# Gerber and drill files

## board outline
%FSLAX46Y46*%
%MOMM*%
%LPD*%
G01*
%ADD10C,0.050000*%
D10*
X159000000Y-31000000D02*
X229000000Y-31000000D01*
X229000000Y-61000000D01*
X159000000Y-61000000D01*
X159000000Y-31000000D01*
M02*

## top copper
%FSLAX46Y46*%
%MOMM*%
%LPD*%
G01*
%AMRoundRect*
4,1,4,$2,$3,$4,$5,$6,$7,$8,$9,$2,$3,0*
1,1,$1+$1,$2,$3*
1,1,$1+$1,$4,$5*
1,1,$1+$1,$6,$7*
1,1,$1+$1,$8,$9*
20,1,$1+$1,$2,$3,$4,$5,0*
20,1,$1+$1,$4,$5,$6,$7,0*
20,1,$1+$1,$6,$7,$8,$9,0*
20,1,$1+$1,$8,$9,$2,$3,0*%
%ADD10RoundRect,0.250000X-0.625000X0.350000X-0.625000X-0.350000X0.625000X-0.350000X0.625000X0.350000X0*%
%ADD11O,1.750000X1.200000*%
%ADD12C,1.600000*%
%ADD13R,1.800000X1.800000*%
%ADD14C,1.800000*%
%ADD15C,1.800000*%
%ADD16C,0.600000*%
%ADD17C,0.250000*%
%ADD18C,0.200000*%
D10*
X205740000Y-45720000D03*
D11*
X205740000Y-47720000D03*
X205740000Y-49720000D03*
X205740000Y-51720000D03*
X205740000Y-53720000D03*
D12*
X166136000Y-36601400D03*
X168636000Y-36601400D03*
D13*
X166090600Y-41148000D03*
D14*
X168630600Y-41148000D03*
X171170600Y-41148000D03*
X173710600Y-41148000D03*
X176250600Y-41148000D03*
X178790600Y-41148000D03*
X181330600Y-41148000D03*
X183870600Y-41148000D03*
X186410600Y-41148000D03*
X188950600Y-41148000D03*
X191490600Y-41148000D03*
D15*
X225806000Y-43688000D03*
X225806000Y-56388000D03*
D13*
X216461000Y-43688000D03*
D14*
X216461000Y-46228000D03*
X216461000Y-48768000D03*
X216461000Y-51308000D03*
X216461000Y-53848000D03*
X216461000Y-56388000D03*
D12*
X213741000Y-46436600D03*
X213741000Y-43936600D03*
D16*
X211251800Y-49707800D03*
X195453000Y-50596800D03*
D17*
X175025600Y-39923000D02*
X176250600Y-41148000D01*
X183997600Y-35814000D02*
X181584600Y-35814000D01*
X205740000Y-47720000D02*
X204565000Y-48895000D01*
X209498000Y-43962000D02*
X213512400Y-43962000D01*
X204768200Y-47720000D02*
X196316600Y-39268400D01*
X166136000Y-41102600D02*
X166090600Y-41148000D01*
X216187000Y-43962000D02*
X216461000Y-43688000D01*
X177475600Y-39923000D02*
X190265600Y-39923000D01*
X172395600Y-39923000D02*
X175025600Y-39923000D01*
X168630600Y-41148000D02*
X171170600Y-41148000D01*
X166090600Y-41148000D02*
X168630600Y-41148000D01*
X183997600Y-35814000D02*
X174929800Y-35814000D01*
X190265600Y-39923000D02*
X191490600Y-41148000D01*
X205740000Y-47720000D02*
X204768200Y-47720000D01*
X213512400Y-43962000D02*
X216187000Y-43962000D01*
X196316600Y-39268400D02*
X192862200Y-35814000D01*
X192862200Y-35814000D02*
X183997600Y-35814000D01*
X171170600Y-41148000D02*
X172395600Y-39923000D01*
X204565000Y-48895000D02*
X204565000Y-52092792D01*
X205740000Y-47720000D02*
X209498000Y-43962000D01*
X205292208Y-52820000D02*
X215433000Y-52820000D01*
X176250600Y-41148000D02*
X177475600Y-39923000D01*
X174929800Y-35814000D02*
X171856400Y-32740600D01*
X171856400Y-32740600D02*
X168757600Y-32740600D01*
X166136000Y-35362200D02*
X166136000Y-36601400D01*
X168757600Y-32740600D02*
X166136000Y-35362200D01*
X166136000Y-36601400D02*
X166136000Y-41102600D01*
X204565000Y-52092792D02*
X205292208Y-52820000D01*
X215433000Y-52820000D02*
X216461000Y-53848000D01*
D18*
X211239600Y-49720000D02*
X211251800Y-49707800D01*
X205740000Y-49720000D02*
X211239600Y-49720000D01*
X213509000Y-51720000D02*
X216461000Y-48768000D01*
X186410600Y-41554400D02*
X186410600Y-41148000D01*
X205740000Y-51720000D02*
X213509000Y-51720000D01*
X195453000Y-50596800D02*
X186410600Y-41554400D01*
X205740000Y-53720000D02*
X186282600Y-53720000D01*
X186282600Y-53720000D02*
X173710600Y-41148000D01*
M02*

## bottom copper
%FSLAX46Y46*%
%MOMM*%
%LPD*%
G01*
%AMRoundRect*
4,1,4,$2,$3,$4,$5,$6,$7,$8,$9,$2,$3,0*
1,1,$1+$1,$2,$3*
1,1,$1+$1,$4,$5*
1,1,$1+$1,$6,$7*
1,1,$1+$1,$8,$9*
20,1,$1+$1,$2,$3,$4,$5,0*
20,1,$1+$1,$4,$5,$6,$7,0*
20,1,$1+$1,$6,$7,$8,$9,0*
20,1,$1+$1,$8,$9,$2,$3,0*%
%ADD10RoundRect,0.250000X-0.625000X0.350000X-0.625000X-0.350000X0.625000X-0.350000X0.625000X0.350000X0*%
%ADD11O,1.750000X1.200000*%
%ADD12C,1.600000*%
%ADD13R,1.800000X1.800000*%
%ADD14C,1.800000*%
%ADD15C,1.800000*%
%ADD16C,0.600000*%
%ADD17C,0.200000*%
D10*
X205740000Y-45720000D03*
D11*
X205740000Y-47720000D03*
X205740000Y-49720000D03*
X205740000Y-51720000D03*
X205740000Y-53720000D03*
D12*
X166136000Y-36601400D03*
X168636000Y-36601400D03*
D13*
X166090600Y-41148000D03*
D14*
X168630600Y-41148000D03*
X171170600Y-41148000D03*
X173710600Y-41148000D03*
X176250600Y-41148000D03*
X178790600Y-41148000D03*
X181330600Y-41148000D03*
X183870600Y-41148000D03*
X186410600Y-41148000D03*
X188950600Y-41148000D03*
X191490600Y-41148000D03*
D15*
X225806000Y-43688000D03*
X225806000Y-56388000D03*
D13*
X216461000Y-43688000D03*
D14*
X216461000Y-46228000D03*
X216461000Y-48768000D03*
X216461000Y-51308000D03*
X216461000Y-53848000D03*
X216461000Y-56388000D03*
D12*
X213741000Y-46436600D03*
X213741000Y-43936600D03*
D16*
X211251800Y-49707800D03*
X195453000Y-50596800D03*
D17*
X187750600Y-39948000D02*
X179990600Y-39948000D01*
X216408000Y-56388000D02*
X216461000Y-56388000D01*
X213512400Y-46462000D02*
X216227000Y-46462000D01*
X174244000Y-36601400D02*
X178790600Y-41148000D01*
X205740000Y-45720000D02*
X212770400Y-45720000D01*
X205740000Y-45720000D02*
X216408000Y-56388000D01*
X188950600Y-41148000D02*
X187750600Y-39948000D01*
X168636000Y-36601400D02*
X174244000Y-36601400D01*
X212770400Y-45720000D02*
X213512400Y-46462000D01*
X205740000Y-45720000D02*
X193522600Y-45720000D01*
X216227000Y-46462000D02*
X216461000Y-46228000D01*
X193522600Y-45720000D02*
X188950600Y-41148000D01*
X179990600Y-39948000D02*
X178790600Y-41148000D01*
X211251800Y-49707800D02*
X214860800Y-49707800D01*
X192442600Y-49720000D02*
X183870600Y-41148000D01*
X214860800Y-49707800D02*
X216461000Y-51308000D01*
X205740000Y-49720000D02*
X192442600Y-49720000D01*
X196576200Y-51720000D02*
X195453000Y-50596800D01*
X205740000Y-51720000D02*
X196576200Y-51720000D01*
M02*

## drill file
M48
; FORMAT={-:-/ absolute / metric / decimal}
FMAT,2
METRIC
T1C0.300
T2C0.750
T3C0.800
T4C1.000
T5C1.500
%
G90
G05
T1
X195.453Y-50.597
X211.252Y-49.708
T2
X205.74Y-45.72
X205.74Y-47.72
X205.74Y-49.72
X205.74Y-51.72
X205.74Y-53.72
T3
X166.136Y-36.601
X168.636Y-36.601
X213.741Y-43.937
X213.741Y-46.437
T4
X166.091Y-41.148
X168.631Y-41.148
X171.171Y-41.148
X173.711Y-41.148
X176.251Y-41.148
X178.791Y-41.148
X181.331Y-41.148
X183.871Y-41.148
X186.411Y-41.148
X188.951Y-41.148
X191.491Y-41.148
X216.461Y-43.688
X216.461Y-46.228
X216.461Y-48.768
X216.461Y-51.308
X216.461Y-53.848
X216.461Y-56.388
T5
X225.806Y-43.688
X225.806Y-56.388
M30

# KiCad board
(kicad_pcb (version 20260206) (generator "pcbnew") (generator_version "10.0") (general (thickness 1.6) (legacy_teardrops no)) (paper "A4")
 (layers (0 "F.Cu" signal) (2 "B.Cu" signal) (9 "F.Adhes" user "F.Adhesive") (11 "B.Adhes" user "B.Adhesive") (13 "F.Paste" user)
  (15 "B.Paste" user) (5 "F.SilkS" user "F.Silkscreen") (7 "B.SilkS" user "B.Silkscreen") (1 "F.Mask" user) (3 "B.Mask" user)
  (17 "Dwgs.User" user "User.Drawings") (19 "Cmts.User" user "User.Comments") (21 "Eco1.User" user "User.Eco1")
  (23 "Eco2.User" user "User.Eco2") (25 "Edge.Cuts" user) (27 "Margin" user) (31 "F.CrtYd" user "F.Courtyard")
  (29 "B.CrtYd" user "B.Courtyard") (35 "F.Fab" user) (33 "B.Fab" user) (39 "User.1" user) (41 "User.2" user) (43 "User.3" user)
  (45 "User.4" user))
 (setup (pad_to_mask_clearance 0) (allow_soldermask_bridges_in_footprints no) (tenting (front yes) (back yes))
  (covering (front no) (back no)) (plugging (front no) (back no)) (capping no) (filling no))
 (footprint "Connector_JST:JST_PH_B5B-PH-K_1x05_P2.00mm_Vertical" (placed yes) (layer "F.Cu") (at 205.74 45.72 -90)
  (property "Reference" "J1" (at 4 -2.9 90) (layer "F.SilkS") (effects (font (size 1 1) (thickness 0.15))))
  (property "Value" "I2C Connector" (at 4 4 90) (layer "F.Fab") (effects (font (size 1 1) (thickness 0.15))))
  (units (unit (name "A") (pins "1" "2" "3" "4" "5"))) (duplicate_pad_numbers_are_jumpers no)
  (pad "1" thru_hole roundrect (at 0 0 270) (size 1.2 1.75) (drill 0.75) (layers "*.Cu" "*.Mask") (remove_unused_layers no)
   (roundrect_rratio 0.208333) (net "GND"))
  (pad "2" thru_hole oval (at 2 0 270) (size 1.2 1.75) (drill 0.75) (layers "*.Cu" "*.Mask") (remove_unused_layers no) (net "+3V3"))
  (pad "3" thru_hole oval (at 4 0 270) (size 1.2 1.75) (drill 0.75) (layers "*.Cu" "*.Mask") (remove_unused_layers no) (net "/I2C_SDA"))
  (pad "4" thru_hole oval (at 6 0 270) (size 1.2 1.75) (drill 0.75) (layers "*.Cu" "*.Mask") (remove_unused_layers no) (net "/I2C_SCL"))
  (pad "5" thru_hole oval (at 8 0 270) (size 1.2 1.75) (drill 0.75) (layers "*.Cu" "*.Mask") (remove_unused_layers no) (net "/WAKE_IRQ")))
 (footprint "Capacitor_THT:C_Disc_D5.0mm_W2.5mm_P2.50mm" (layer "F.Cu") (at 166.136 36.6014)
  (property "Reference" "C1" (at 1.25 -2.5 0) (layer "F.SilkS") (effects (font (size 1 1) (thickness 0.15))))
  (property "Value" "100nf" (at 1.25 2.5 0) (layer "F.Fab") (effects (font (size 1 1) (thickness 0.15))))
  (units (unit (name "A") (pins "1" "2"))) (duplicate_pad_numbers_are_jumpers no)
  (pad "1" thru_hole circle (at 0 0) (size 1.6 1.6) (drill 0.8) (layers "*.Cu" "*.Mask") (remove_unused_layers no) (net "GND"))
  (pad "2" thru_hole circle (at 2.5 0) (size 1.6 1.6) (drill 0.8) (layers "*.Cu" "*.Mask") (remove_unused_layers no) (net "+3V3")))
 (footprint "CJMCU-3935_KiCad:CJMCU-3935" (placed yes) (layer "F.Cu") (at 178.7906 41.148)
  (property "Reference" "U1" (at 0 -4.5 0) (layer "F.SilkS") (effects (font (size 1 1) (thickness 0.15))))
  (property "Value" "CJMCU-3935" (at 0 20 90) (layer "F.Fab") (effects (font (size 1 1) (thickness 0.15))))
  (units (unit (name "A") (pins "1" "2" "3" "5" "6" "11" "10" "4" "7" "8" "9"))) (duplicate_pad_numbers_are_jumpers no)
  (pad "1" thru_hole rect (at -12.7 0) (size 1.8 1.8) (drill 1) (layers "*.Cu" "*.Mask") (remove_unused_layers no) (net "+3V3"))
  (pad "2" thru_hole circle (at -10.16 0) (size 1.8 1.8) (drill 1) (layers "*.Cu" "*.Mask") (remove_unused_layers no) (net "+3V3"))
  (pad "3" thru_hole circle (at -7.62 0) (size 1.8 1.8) (drill 1) (layers "*.Cu" "*.Mask") (remove_unused_layers no) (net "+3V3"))
  (pad "4" thru_hole circle (at -5.08 0) (size 1.8 1.8) (drill 1) (layers "*.Cu" "*.Mask") (remove_unused_layers no) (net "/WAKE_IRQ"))
  (pad "5" thru_hole circle (at -2.54 0) (size 1.8 1.8) (drill 1) (layers "*.Cu" "*.Mask") (remove_unused_layers no) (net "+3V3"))
  (pad "6" thru_hole circle (at 0 0) (size 1.8 1.8) (drill 1) (layers "*.Cu" "*.Mask") (remove_unused_layers no) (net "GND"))
  (pad "7" thru_hole circle (at 2.54 0) (size 1.8 1.8) (drill 1) (layers "*.Cu" "*.Mask") (remove_unused_layers no)
   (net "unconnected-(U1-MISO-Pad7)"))
  (pad "8" thru_hole circle (at 5.08 0) (size 1.8 1.8) (drill 1) (layers "*.Cu" "*.Mask") (remove_unused_layers no) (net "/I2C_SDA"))
  (pad "9" thru_hole circle (at 7.62 0) (size 1.8 1.8) (drill 1) (layers "*.Cu" "*.Mask") (remove_unused_layers no) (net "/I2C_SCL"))
  (pad "10" thru_hole circle (at 10.16 0) (size 1.8 1.8) (drill 1) (layers "*.Cu" "*.Mask") (remove_unused_layers no) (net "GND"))
  (pad "11" thru_hole circle (at 12.7 0) (size 1.8 1.8) (drill 1) (layers "*.Cu" "*.Mask") (remove_unused_layers no) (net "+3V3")))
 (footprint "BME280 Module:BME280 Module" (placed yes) (layer "F.Cu") (at 216.461 43.688 -90)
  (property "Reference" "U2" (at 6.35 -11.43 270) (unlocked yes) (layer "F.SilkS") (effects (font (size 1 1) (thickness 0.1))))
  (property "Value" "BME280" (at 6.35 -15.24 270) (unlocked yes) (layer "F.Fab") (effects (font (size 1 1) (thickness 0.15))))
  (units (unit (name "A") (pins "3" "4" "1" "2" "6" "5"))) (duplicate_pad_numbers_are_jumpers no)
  (pad "" np_thru_hole circle (at 0 -9.345 270) (size 1.8 1.8) (drill 1.5) (layers "*.Cu" "*.Mask"))
  (pad "" np_thru_hole circle (at 12.7 -9.345 270) (size 1.8 1.8) (drill 1.5) (layers "*.Cu" "*.Mask"))
  (pad "1" thru_hole rect (at 0 0 270) (size 1.8 1.8) (drill 1) (layers "*.Cu" "*.Mask") (remove_unused_layers no) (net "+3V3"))
  (pad "2" thru_hole circle (at 2.54 0 270) (size 1.8 1.8) (drill 1) (layers "*.Cu" "*.Mask") (remove_unused_layers no) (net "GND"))
  (pad "3" thru_hole circle (at 5.08 0 270) (size 1.8 1.8) (drill 1) (layers "*.Cu" "*.Mask") (remove_unused_layers no) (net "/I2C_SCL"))
  (pad "4" thru_hole circle (at 7.62 0 270) (size 1.8 1.8) (drill 1) (layers "*.Cu" "*.Mask") (remove_unused_layers no) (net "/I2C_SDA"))
  (pad "5" thru_hole circle (at 10.16 0 270) (size 1.8 1.8) (drill 1) (layers "*.Cu" "*.Mask") (remove_unused_layers no) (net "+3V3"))
  (pad "6" thru_hole circle (at 12.7 0 270) (size 1.8 1.8) (drill 1) (layers "*.Cu" "*.Mask") (remove_unused_layers no) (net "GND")))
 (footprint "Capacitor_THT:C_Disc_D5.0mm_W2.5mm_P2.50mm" (layer "F.Cu") (at 213.741 46.4366 90)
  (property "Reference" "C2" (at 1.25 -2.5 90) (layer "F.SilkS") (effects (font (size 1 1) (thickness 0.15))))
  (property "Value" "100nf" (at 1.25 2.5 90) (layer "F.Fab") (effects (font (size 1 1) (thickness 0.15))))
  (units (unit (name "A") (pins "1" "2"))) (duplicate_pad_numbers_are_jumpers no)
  (pad "1" thru_hole circle (at 0 0 90) (size 1.6 1.6) (drill 0.8) (layers "*.Cu" "*.Mask") (remove_unused_layers no) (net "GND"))
  (pad "2" thru_hole circle (at 2.5 0 90) (size 1.6 1.6) (drill 0.8) (layers "*.Cu" "*.Mask") (remove_unused_layers no) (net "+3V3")))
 (gr_rect (start 159 31) (end 229 61) (stroke (width 0.05) (type default)) (fill no) (layer "Edge.Cuts"))
 (segment (start 187.7506 39.948) (end 179.9906 39.948) (width 0.2) (layer "B.Cu") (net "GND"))
 (segment (start 216.408 56.388) (end 216.461 56.388) (width 0.2) (layer "B.Cu") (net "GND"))
 (segment (start 213.5124 46.462) (end 216.227 46.462) (width 0.2) (layer "B.Cu") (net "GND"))
 (segment (start 174.244 36.6014) (end 178.7906 41.148) (width 0.2) (layer "B.Cu") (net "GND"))
 (segment (start 205.74 45.72) (end 212.7704 45.72) (width 0.2) (layer "B.Cu") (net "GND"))
 (segment (start 205.74 45.72) (end 216.408 56.388) (width 0.2) (layer "B.Cu") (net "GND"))
 (segment (start 188.9506 41.148) (end 187.7506 39.948) (width 0.2) (layer "B.Cu") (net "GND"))
 (segment (start 168.636 36.6014) (end 174.244 36.6014) (width 0.2) (layer "B.Cu") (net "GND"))
 (segment (start 212.7704 45.72) (end 213.5124 46.462) (width 0.2) (layer "B.Cu") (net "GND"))
 (segment (start 205.74 45.72) (end 193.5226 45.72) (width 0.2) (layer "B.Cu") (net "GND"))
 (segment (start 216.227 46.462) (end 216.461 46.228) (width 0.2) (layer "B.Cu") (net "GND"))
 (segment (start 193.5226 45.72) (end 188.9506 41.148) (width 0.2) (layer "B.Cu") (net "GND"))
 (segment (start 179.9906 39.948) (end 178.7906 41.148) (width 0.2) (layer "B.Cu") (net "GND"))
 (segment (start 175.0256 39.923) (end 176.2506 41.148) (width 0.25) (layer "F.Cu") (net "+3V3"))
 (segment (start 183.9976 35.814) (end 181.5846 35.814) (width 0.25) (layer "F.Cu") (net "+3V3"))
 (segment (start 205.74 47.72) (end 204.565 48.895) (width 0.25) (layer "F.Cu") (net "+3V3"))
 (segment (start 209.498 43.962) (end 213.5124 43.962) (width 0.25) (layer "F.Cu") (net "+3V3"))
 (segment (start 204.7682 47.72) (end 196.3166 39.2684) (width 0.25) (layer "F.Cu") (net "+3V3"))
 (segment (start 166.136 41.1026) (end 166.0906 41.148) (width 0.25) (layer "F.Cu") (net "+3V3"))
 (segment (start 216.187 43.962) (end 216.461 43.688) (width 0.25) (layer "F.Cu") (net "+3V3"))
 (segment (start 177.4756 39.923) (end 190.2656 39.923) (width 0.25) (layer "F.Cu") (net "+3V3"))
 (segment (start 172.3956 39.923) (end 175.0256 39.923) (width 0.25) (layer "F.Cu") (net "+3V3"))
 (segment (start 168.6306 41.148) (end 171.1706 41.148) (width 0.25) (layer "F.Cu") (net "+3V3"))
 (segment (start 166.0906 41.148) (end 168.6306 41.148) (width 0.25) (layer "F.Cu") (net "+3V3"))
 (segment (start 183.9976 35.814) (end 174.9298 35.814) (width 0.25) (layer "F.Cu") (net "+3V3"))
 (segment (start 190.2656 39.923) (end 191.4906 41.148) (width 0.25) (layer "F.Cu") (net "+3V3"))
 (segment (start 205.74 47.72) (end 204.7682 47.72) (width 0.25) (layer "F.Cu") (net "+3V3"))
 (segment (start 213.5124 43.962) (end 216.187 43.962) (width 0.25) (layer "F.Cu") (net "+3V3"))
 (segment (start 196.3166 39.2684) (end 192.8622 35.814) (width 0.25) (layer "F.Cu") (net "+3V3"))
 (segment (start 192.8622 35.814) (end 183.9976 35.814) (width 0.25) (layer "F.Cu") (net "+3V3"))
 (segment (start 171.1706 41.148) (end 172.3956 39.923) (width 0.25) (layer "F.Cu") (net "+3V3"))
 (segment (start 204.565 48.895) (end 204.565 52.092792) (width 0.25) (layer "F.Cu") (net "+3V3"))
 (segment (start 205.74 47.72) (end 209.498 43.962) (width 0.25) (layer "F.Cu") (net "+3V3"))
 (segment (start 205.292208 52.82) (end 215.433 52.82) (width 0.25) (layer "F.Cu") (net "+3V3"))
 (segment (start 176.2506 41.148) (end 177.4756 39.923) (width 0.25) (layer "F.Cu") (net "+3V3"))
 (segment (start 174.9298 35.814) (end 171.8564 32.7406) (width 0.25) (layer "F.Cu") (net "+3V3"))
 (segment (start 171.8564 32.7406) (end 168.7576 32.7406) (width 0.25) (layer "F.Cu") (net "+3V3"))
 (segment (start 166.136 35.3622) (end 166.136 36.6014) (width 0.25) (layer "F.Cu") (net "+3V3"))
 (segment (start 168.7576 32.7406) (end 166.136 35.3622) (width 0.25) (layer "F.Cu") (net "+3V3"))
 (segment (start 166.136 36.6014) (end 166.136 41.1026) (width 0.25) (layer "F.Cu") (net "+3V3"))
 (segment (start 204.565 52.092792) (end 205.292208 52.82) (width 0.25) (layer "F.Cu") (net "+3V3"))
 (segment (start 215.433 52.82) (end 216.461 53.848) (width 0.25) (layer "F.Cu") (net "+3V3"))
 (segment (start 211.2396 49.72) (end 211.2518 49.7078) (width 0.2) (layer "F.Cu") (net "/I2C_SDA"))
 (segment (start 205.74 49.72) (end 211.2396 49.72) (width 0.2) (layer "F.Cu") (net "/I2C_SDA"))
 (via (at 211.2518 49.7078) (size 0.6) (drill 0.3) (layers "F.Cu" "B.Cu") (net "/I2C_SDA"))
 (segment (start 211.2518 49.7078) (end 214.8608 49.7078) (width 0.2) (layer "B.Cu") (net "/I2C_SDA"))
 (segment (start 192.4426 49.72) (end 183.8706 41.148) (width 0.2) (layer "B.Cu") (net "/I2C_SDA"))
 (segment (start 214.8608 49.7078) (end 216.461 51.308) (width 0.2) (layer "B.Cu") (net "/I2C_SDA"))
 (segment (start 205.74 49.72) (end 192.4426 49.72) (width 0.2) (layer "B.Cu") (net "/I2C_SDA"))
 (segment (start 213.509 51.72) (end 216.461 48.768) (width 0.2) (layer "F.Cu") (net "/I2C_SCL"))
 (segment (start 186.4106 41.5544) (end 186.4106 41.148) (width 0.2) (layer "F.Cu") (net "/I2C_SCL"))
 (segment (start 205.74 51.72) (end 213.509 51.72) (width 0.2) (layer "F.Cu") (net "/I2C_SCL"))
 (segment (start 195.453 50.5968) (end 186.4106 41.5544) (width 0.2) (layer "F.Cu") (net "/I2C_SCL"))
 (via (at 195.453 50.5968) (size 0.6) (drill 0.3) (layers "F.Cu" "B.Cu") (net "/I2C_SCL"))
 (segment (start 196.5762 51.72) (end 195.453 50.5968) (width 0.2) (layer "B.Cu") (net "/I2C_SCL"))
 (segment (start 205.74 51.72) (end 196.5762 51.72) (width 0.2) (layer "B.Cu") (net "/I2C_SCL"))
 (segment (start 205.74 53.72) (end 186.2826 53.72) (width 0.2) (layer "F.Cu") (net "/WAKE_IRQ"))
 (segment (start 186.2826 53.72) (end 173.7106 41.148) (width 0.2) (layer "F.Cu") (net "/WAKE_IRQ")))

